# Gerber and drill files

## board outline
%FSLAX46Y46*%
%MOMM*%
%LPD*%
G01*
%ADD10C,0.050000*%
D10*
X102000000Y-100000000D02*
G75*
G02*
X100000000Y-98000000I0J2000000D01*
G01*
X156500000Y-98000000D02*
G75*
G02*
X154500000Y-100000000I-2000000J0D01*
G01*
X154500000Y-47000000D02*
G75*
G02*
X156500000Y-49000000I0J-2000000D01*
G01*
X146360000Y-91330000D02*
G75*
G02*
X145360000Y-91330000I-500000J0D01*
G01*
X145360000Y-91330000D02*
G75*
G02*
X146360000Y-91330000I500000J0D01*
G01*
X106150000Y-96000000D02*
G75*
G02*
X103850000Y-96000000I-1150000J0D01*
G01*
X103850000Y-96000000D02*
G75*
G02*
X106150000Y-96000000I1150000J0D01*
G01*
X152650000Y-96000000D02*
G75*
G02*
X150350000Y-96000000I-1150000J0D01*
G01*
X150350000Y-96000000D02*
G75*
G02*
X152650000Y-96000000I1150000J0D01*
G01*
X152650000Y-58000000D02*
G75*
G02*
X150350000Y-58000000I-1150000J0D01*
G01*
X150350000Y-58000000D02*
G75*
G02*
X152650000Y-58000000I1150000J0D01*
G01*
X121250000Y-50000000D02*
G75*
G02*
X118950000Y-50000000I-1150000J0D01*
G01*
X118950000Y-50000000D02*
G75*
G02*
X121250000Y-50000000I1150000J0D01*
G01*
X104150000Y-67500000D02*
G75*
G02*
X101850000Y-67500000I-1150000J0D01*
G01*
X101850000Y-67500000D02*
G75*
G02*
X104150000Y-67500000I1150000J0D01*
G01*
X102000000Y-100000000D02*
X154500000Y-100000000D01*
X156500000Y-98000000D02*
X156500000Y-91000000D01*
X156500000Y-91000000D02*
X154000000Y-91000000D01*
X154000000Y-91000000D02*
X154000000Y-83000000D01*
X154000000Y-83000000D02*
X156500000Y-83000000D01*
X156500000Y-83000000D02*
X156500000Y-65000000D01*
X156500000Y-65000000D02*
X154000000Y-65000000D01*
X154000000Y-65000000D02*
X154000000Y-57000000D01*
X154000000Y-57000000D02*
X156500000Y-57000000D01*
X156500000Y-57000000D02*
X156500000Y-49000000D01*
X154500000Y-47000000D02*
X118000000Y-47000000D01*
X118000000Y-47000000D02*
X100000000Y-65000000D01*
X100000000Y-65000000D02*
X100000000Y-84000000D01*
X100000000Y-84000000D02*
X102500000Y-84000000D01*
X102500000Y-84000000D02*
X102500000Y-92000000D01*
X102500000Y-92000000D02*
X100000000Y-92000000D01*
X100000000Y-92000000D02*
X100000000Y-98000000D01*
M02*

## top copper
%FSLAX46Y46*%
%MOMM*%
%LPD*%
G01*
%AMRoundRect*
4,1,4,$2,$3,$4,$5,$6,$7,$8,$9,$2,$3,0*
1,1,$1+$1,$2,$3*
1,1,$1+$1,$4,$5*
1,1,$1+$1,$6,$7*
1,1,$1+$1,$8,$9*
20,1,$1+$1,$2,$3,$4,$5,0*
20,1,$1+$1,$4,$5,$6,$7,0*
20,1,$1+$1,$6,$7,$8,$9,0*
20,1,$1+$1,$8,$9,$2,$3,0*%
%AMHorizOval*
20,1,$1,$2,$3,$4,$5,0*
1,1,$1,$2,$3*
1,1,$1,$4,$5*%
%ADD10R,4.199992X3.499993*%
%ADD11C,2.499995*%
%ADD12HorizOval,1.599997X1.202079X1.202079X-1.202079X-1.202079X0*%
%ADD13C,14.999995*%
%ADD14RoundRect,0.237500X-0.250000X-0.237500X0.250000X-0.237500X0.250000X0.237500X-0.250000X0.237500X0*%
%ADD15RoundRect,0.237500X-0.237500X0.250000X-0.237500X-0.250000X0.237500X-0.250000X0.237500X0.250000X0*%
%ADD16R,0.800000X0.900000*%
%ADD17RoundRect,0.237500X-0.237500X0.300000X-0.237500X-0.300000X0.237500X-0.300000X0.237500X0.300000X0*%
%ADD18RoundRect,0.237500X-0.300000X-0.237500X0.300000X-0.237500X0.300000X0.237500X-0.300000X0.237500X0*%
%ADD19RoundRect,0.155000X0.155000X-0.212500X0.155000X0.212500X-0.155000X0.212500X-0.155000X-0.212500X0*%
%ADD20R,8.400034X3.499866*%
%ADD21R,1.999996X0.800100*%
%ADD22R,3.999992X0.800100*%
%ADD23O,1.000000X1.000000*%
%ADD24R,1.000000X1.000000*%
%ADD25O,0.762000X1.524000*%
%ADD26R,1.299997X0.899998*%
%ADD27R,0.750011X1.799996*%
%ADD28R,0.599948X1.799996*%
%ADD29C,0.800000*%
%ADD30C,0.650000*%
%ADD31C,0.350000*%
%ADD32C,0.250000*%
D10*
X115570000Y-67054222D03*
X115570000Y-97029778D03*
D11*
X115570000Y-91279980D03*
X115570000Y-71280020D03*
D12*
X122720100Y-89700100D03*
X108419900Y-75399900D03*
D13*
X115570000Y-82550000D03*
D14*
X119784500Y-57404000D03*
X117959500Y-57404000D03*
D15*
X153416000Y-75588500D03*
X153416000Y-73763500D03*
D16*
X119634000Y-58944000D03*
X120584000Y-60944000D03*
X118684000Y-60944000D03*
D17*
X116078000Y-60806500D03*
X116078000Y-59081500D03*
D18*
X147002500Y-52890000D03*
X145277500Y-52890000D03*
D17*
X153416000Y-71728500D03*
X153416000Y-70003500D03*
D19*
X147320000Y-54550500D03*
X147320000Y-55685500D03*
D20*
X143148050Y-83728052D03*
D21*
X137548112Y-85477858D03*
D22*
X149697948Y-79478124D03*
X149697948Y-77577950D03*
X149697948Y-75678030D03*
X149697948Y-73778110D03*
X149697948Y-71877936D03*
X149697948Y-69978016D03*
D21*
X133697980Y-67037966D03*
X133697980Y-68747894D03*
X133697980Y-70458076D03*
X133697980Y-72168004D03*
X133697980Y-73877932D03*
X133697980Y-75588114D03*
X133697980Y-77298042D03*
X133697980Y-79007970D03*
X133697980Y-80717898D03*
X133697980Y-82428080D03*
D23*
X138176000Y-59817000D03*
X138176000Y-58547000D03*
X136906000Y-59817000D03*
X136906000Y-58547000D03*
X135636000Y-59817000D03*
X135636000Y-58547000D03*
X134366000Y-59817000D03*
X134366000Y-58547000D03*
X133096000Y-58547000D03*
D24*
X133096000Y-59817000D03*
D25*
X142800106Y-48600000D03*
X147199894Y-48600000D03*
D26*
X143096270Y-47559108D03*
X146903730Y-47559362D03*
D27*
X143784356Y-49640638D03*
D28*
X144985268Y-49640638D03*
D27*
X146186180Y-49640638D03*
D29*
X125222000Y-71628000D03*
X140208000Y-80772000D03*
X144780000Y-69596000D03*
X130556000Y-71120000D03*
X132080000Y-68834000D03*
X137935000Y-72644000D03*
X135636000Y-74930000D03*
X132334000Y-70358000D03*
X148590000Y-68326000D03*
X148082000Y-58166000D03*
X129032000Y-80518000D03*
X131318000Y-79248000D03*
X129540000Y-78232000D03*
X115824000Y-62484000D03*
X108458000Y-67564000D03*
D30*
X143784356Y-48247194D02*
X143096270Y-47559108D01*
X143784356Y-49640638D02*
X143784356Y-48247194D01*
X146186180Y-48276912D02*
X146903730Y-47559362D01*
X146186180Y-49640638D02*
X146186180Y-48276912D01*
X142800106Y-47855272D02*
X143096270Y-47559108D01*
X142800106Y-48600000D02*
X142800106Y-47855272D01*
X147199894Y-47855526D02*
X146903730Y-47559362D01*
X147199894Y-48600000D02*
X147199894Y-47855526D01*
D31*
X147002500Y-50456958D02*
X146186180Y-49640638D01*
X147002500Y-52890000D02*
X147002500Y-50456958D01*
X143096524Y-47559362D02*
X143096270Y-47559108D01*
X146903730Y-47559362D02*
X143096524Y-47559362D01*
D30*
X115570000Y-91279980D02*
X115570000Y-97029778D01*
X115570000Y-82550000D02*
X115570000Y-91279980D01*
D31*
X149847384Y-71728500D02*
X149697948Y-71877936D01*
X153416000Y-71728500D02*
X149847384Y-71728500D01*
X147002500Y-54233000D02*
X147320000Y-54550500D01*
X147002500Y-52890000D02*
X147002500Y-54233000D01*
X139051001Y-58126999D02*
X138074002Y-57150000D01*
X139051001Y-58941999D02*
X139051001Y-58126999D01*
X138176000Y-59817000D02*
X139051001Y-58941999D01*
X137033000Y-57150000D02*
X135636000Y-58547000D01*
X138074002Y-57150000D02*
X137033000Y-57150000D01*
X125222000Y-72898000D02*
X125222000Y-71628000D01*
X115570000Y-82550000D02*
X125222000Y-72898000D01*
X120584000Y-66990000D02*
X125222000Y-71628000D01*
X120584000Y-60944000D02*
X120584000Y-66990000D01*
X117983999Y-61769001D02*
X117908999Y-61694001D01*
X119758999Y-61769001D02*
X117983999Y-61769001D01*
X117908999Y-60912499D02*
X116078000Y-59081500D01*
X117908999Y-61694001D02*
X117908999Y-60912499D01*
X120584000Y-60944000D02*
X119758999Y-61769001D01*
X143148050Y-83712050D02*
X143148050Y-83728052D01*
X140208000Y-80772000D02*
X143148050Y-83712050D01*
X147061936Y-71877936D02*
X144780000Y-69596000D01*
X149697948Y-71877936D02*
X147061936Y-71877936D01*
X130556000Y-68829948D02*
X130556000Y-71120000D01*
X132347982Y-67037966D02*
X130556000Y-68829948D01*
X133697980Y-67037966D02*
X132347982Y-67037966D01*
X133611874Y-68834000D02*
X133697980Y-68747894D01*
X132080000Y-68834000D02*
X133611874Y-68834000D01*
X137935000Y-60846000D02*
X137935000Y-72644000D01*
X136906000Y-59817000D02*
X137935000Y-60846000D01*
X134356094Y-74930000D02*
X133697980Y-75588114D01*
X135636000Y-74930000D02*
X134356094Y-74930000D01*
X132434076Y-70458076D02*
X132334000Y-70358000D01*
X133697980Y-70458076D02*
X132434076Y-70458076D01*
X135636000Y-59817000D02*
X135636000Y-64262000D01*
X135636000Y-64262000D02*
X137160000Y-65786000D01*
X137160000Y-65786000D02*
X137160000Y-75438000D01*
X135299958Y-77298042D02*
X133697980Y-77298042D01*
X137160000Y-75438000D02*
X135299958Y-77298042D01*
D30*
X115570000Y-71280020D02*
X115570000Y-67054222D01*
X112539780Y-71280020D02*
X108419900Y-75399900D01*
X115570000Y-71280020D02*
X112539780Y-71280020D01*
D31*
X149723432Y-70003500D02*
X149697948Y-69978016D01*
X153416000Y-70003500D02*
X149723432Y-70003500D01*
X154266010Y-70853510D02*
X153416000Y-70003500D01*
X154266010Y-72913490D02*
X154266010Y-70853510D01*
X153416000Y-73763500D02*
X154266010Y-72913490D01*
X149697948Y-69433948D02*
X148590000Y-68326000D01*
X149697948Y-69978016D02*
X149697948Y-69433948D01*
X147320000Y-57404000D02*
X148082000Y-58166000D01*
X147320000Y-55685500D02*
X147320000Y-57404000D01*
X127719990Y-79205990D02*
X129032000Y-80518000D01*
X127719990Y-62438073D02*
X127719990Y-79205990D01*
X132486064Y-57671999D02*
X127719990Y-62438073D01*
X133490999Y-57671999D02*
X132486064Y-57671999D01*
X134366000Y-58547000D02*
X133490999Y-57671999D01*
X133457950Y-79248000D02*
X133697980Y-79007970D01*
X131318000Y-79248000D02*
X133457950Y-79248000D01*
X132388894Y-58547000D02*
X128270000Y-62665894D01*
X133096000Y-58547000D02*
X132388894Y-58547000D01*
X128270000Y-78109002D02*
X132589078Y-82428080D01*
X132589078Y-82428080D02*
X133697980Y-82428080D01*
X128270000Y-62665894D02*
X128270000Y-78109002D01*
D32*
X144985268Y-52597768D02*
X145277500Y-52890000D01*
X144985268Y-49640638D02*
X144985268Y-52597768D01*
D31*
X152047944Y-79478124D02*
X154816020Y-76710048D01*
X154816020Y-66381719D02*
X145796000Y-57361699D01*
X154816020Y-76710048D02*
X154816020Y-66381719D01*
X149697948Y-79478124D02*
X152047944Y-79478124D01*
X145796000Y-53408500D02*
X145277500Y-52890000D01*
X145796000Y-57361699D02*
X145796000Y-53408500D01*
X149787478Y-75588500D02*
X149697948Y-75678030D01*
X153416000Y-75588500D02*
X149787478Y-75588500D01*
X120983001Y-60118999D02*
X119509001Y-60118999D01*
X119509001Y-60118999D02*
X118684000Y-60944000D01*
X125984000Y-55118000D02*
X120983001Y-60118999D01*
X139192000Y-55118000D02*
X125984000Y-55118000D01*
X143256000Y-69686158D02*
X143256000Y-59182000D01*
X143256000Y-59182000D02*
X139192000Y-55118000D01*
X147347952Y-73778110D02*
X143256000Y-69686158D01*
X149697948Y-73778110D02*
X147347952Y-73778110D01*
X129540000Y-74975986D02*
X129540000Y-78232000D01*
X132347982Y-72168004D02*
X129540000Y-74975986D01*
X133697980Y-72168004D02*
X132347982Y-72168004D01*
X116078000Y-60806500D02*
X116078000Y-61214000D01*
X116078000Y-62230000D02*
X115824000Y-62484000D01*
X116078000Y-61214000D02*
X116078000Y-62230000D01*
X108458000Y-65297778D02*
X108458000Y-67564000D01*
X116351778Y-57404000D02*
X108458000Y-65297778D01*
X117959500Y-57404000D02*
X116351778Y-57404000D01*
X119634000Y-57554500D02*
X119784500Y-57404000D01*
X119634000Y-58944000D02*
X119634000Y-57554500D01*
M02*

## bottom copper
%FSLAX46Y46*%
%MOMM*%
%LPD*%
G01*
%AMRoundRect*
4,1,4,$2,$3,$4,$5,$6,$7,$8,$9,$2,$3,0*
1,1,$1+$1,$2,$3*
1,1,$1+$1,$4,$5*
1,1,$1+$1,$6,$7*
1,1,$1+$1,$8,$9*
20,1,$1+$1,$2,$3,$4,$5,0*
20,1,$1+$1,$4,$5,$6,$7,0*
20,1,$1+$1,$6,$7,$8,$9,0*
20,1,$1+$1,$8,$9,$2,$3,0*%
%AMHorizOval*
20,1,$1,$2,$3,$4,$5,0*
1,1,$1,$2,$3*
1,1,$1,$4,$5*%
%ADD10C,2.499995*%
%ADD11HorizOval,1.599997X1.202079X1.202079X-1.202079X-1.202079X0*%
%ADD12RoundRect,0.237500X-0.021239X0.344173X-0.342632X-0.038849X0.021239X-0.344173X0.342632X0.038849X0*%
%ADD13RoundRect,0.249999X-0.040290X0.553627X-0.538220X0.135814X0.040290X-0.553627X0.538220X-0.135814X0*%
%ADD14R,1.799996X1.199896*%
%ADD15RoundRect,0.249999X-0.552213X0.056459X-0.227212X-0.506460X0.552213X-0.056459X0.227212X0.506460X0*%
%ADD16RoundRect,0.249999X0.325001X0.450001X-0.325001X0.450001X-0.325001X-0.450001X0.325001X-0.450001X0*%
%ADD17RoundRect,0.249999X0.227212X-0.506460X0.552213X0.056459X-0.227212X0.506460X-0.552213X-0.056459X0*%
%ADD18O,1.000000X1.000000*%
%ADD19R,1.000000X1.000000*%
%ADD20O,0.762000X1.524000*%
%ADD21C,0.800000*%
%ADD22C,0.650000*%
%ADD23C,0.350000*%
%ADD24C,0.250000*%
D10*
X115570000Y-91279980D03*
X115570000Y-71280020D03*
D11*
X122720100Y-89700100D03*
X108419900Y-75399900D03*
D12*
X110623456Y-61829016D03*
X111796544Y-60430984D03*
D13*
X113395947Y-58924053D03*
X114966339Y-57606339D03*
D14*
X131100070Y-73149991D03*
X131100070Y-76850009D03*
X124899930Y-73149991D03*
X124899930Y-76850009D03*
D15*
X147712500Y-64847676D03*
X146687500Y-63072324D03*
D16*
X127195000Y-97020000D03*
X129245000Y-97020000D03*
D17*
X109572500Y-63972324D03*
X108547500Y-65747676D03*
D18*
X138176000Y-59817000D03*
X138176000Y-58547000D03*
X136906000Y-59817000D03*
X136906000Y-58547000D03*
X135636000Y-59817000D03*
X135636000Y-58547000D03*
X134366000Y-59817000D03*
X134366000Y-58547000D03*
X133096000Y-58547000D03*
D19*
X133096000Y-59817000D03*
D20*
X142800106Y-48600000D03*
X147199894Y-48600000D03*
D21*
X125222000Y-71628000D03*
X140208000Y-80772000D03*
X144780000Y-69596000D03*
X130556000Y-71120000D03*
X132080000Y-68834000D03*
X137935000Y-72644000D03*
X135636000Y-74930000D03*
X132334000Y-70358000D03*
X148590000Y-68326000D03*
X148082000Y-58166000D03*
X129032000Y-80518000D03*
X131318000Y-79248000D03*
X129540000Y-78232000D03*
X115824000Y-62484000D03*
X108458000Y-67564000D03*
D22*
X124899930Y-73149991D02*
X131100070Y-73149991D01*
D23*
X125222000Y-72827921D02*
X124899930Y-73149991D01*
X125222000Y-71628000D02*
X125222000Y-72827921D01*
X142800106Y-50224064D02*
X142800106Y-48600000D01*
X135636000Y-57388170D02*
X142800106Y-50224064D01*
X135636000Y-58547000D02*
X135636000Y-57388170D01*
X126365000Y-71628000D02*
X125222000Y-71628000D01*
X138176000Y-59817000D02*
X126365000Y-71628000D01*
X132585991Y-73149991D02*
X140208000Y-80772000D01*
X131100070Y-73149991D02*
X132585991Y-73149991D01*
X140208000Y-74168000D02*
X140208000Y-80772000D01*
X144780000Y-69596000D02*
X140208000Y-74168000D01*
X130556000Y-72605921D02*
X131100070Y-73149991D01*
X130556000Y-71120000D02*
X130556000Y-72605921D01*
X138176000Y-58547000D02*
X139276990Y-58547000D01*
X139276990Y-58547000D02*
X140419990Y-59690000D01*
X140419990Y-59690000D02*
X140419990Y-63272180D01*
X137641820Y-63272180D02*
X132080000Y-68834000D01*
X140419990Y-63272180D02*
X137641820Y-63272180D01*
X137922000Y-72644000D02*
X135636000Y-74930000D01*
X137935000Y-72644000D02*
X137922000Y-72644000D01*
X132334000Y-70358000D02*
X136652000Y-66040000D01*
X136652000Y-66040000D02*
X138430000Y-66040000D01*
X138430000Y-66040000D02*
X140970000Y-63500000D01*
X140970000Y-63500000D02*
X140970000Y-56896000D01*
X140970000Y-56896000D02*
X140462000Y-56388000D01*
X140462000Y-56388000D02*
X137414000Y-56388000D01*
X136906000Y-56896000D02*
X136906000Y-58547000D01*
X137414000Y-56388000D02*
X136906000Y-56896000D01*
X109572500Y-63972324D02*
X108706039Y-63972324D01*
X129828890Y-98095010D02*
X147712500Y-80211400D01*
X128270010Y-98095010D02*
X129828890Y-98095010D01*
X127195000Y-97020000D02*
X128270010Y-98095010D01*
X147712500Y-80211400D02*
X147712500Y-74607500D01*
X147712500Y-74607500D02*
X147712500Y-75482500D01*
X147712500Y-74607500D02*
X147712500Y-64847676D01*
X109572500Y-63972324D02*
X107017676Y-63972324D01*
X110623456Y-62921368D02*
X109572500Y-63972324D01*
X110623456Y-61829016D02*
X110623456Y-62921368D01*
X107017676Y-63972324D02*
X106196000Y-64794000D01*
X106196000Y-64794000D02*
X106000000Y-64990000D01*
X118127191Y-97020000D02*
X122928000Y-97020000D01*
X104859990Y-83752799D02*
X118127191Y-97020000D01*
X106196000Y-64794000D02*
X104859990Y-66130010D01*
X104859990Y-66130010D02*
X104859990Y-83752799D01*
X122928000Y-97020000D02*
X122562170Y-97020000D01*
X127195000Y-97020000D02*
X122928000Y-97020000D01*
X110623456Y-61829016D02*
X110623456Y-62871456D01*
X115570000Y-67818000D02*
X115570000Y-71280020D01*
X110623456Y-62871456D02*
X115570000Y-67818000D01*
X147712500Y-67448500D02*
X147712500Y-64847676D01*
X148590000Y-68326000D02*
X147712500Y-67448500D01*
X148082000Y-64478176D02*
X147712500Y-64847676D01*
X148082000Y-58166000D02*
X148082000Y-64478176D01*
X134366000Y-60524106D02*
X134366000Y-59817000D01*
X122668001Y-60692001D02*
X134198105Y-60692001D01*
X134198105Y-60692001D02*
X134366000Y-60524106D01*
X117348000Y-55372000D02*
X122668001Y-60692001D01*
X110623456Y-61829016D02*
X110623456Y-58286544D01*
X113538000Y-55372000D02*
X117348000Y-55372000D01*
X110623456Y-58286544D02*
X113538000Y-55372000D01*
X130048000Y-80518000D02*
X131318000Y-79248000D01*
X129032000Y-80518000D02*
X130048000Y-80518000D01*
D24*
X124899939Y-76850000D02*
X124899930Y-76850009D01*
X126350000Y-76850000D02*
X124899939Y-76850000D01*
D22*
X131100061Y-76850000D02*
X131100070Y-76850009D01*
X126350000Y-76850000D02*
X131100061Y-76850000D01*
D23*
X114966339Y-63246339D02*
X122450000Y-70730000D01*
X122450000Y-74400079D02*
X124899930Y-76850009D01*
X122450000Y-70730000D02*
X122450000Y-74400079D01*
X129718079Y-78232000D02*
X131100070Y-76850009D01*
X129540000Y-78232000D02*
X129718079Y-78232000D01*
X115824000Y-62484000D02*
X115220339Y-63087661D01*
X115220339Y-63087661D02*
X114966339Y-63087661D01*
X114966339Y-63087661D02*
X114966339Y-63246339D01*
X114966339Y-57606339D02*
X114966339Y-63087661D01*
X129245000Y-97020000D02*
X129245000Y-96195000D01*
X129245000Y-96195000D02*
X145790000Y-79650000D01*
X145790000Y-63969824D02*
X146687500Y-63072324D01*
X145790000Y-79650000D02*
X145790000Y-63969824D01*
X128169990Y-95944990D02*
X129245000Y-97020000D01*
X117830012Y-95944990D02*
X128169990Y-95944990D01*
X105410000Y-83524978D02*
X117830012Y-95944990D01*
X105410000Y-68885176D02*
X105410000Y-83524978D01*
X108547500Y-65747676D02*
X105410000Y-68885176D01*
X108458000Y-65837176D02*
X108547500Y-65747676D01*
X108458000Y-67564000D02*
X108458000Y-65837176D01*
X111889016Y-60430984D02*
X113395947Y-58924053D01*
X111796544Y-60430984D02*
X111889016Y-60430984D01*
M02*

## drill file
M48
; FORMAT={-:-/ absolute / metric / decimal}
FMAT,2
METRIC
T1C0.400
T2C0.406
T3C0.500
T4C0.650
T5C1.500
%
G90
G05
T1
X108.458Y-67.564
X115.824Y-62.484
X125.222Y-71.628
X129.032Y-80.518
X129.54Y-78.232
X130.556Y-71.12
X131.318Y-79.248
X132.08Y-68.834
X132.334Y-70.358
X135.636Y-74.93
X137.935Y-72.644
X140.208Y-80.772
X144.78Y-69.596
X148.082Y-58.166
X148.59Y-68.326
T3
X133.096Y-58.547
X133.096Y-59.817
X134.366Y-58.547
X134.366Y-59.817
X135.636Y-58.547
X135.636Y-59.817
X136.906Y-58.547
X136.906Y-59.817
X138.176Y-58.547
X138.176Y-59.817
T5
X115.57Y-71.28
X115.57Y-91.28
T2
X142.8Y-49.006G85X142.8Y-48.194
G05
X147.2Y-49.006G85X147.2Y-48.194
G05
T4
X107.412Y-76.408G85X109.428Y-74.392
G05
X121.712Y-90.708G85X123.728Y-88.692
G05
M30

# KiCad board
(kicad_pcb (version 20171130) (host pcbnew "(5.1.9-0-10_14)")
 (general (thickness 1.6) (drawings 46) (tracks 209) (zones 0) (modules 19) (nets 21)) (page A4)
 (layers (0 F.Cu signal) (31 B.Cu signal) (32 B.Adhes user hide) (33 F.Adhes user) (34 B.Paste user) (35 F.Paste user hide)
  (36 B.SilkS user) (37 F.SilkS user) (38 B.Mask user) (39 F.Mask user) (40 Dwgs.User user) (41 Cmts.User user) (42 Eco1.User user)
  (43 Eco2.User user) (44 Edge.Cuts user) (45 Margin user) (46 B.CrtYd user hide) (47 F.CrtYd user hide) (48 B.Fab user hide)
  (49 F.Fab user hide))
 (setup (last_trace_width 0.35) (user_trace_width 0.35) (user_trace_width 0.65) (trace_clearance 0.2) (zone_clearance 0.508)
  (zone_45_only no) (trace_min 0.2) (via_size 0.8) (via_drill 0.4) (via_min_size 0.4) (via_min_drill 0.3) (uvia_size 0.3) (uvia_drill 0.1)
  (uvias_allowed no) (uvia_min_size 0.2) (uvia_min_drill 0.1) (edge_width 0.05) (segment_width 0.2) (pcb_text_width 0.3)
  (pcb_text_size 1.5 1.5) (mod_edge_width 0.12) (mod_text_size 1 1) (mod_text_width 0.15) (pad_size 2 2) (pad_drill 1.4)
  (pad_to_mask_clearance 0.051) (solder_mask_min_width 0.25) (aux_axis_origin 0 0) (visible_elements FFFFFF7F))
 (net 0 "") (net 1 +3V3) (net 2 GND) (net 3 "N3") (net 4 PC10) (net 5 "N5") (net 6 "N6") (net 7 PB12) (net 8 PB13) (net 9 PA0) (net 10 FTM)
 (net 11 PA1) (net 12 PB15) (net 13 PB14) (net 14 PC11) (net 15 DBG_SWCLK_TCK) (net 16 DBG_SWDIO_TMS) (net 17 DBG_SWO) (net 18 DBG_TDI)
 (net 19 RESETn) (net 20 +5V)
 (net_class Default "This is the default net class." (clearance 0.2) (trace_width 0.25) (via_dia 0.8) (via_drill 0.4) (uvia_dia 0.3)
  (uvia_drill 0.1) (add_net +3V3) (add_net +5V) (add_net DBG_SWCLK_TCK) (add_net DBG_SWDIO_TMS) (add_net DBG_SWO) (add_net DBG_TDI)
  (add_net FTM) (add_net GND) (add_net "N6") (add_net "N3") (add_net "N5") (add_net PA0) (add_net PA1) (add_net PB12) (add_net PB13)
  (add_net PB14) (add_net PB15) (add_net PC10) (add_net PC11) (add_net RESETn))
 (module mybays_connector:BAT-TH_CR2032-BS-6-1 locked (layer F.Cu) (at 115.57 82.042 90)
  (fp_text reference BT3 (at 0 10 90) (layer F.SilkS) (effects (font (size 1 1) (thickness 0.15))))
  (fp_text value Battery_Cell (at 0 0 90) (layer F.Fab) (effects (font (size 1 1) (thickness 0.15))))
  (pad 1 smd rect (at 14.987778 0 90) (size 3.499993 4.199992) (layers F.Cu F.Paste F.Mask) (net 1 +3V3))
  (pad 2 smd rect (at -14.987778 0 90) (size 3.499993 4.199992) (layers F.Cu F.Paste F.Mask) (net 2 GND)))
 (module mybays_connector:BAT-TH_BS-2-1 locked (layer F.Cu) (at 115.57 81.28 180)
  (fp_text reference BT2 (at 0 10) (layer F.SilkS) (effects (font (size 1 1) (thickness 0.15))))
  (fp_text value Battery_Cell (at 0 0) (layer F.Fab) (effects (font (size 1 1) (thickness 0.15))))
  (pad 2 thru_hole circle (at 0 -9.99998 270) (size 2.499995 2.499995) (drill 1.500022) (layers *.Cu *.Mask) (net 2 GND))
  (pad 1 thru_hole circle (at 0 9.99998 270) (size 2.499995 2.499995) (drill 1.500022) (layers *.Cu *.Mask) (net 1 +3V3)))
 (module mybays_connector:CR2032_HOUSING (layer F.Cu) (at 115.57 82.55 90)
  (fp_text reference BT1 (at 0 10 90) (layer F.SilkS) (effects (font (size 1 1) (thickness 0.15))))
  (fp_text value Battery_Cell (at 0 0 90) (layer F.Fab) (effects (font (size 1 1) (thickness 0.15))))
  (pad 3 thru_hole oval (at -7.1501 7.1501 135) (size 1.599997 4.99999) (drill oval 0.649986 3.499968) (layers *.Cu *.Mask))
  (pad 1 thru_hole oval (at 7.1501 -7.1501 135) (size 1.599997 4.99999) (drill oval 0.649986 3.500044) (layers *.Cu *.Mask) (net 1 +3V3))
  (pad 2 smd circle (at 0 0 90) (size 14.999995 14.999995) (layers F.Cu F.Paste F.Mask) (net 2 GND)))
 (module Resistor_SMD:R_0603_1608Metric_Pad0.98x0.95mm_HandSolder (layer B.Cu) (at 111.21 61.13 230)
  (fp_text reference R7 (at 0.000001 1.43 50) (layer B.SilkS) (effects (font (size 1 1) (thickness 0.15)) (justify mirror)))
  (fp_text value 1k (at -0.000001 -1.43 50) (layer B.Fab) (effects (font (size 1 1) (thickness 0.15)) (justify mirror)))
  (pad 2 smd roundrect (at 0.9125 0 230) (size 0.975 0.95) (layers B.Cu B.Paste B.Mask) (roundrect_rratio 0.25) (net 1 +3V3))
  (pad 1 smd roundrect (at -0.9125 0 230) (size 0.975 0.95) (layers B.Cu B.Paste B.Mask) (roundrect_rratio 0.25) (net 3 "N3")))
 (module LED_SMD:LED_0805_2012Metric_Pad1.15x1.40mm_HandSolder (layer B.Cu) (at 114.181143 58.265196 220)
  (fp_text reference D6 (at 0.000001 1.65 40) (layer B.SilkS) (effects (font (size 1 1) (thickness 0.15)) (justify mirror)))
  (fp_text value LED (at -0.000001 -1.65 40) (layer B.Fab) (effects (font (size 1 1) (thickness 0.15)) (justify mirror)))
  (pad 2 smd roundrect (at 1.025 0 220) (size 1.15 1.4) (layers B.Cu B.Paste B.Mask) (roundrect_rratio 0.2173904347826087) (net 3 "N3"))
  (pad 1 smd roundrect (at -1.025 0 220) (size 1.15 1.4) (layers B.Cu B.Paste B.Mask) (roundrect_rratio 0.2173904347826087) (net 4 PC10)))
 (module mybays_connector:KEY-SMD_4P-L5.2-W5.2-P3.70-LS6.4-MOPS (layer B.Cu) (at 128 75)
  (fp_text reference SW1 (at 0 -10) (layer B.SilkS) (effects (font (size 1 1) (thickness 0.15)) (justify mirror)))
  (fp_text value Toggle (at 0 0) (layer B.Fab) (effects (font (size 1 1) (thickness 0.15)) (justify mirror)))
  (pad 4 smd rect (at 3.10007 -1.850009) (size 1.799996 1.199896) (layers B.Cu B.Paste B.Mask) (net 2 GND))
  (pad 3 smd rect (at 3.10007 1.850009) (size 1.799996 1.199896) (layers B.Cu B.Paste B.Mask) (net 4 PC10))
  (pad 2 smd rect (at -3.10007 -1.850009) (size 1.799996 1.199896) (layers B.Cu B.Paste B.Mask) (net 2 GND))
  (pad 1 smd rect (at -3.10007 1.850009) (size 1.799996 1.199896) (layers B.Cu B.Paste B.Mask) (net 4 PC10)))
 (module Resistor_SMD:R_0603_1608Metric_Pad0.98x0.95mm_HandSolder (layer F.Cu) (at 118.872 57.404)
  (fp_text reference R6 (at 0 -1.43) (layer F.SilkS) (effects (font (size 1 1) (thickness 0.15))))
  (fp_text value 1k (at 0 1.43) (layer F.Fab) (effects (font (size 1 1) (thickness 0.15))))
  (pad 2 smd roundrect (at 0.9125 0) (size 0.975 0.95) (layers F.Cu F.Paste F.Mask) (roundrect_rratio 0.25) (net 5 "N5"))
  (pad 1 smd roundrect (at -0.9125 0) (size 0.975 0.95) (layers F.Cu F.Paste F.Mask) (roundrect_rratio 0.25) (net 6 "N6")))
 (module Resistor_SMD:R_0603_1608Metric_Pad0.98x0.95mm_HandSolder (layer F.Cu) (at 153.416 74.676 270)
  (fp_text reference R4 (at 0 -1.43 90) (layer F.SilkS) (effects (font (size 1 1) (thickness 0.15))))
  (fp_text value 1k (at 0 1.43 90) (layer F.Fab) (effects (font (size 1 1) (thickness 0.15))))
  (pad 2 smd roundrect (at 0.9125 0 270) (size 0.975 0.95) (layers F.Cu F.Paste F.Mask) (roundrect_rratio 0.25) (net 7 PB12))
  (pad 1 smd roundrect (at -0.9125 0 270) (size 0.975 0.95) (layers F.Cu F.Paste F.Mask) (roundrect_rratio 0.25) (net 1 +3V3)))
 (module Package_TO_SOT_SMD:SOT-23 (layer F.Cu) (at 119.634 59.944 90)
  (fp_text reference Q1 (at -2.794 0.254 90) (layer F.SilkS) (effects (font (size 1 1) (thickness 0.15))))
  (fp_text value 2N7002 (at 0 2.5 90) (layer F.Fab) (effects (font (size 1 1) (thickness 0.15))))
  (pad 3 smd rect (at 1 0 90) (size 0.9 0.8) (layers F.Cu F.Paste F.Mask) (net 5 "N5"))
  (pad 2 smd rect (at -1 0.95 90) (size 0.9 0.8) (layers F.Cu F.Paste F.Mask) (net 2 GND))
  (pad 1 smd rect (at -1 -0.95 90) (size 0.9 0.8) (layers F.Cu F.Paste F.Mask) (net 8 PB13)))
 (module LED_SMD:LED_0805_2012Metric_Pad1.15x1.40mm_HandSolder (layer B.Cu) (at 147.2 63.96 300)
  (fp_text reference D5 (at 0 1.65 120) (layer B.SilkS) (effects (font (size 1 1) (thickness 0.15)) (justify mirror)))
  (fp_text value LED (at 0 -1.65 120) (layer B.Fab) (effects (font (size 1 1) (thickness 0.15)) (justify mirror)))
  (pad 2 smd roundrect (at 1.025 0 300) (size 1.15 1.4) (layers B.Cu B.Paste B.Mask) (roundrect_rratio 0.2173904347826087) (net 1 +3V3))
  (pad 1 smd roundrect (at -1.025 0 300) (size 1.15 1.4) (layers B.Cu B.Paste B.Mask) (roundrect_rratio 0.2173904347826087) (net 6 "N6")))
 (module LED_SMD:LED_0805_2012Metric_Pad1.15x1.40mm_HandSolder (layer B.Cu) (at 128.22 97.02 180)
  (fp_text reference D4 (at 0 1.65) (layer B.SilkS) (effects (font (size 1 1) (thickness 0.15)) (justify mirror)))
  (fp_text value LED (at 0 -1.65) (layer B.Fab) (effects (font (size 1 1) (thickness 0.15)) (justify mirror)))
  (pad 2 smd roundrect (at 1.025 0 180) (size 1.15 1.4) (layers B.Cu B.Paste B.Mask) (roundrect_rratio 0.2173904347826087) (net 1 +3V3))
  (pad 1 smd roundrect (at -1.025 0 180) (size 1.15 1.4) (layers B.Cu B.Paste B.Mask) (roundrect_rratio 0.2173904347826087) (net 6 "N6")))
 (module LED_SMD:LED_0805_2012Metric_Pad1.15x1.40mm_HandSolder (layer B.Cu) (at 109.06 64.86 60)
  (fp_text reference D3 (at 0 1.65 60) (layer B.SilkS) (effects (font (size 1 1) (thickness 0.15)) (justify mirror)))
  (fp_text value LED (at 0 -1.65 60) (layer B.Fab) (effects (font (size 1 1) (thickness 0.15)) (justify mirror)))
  (pad 2 smd roundrect (at 1.025 0 60) (size 1.15 1.4) (layers B.Cu B.Paste B.Mask) (roundrect_rratio 0.2173904347826087) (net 1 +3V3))
  (pad 1 smd roundrect (at -1.025 0 60) (size 1.15 1.4) (layers B.Cu B.Paste B.Mask) (roundrect_rratio 0.2173904347826087) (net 6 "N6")))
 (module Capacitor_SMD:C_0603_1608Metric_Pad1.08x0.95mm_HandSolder (layer F.Cu) (at 116.078 59.944 270)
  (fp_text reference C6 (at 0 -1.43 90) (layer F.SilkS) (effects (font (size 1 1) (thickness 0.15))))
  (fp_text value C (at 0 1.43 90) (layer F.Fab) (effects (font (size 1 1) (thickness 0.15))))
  (pad 2 smd roundrect (at 0.8625 0 270) (size 1.075 0.95) (layers F.Cu F.Paste F.Mask) (roundrect_rratio 0.25) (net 4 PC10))
  (pad 1 smd roundrect (at -0.8625 0 270) (size 1.075 0.95) (layers F.Cu F.Paste F.Mask) (roundrect_rratio 0.25) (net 2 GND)))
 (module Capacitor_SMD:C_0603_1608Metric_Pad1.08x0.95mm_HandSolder (layer F.Cu) (at 146.14 52.89)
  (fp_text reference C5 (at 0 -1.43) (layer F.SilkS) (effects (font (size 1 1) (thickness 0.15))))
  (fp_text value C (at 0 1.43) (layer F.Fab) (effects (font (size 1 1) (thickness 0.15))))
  (pad 2 smd roundrect (at 0.8625 0) (size 1.075 0.95) (layers F.Cu F.Paste F.Mask) (roundrect_rratio 0.25) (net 2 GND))
  (pad 1 smd roundrect (at -0.8625 0) (size 1.075 0.95) (layers F.Cu F.Paste F.Mask) (roundrect_rratio 0.25) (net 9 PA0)))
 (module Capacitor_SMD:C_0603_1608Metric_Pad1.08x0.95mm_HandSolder (layer F.Cu) (at 153.416 70.866 270)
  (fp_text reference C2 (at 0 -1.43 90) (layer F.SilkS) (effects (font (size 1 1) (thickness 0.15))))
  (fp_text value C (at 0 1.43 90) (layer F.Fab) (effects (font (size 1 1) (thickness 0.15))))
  (pad 2 smd roundrect (at 0.8625 0 270) (size 1.075 0.95) (layers F.Cu F.Paste F.Mask) (roundrect_rratio 0.25) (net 2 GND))
  (pad 1 smd roundrect (at -0.8625 0 270) (size 1.075 0.95) (layers F.Cu F.Paste F.Mask) (roundrect_rratio 0.25) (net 1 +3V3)))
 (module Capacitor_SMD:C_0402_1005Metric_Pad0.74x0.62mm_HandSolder (layer F.Cu) (at 147.32 55.118 90)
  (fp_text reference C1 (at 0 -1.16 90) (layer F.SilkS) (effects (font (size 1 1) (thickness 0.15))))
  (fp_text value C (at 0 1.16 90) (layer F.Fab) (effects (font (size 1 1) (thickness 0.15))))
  (pad 2 smd roundrect (at 0.5675 0 90) (size 0.735 0.62) (layers F.Cu F.Paste F.Mask) (roundrect_rratio 0.25) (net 2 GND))
  (pad 1 smd roundrect (at -0.5675 0 90) (size 0.735 0.62) (layers F.Cu F.Paste F.Mask) (roundrect_rratio 0.25) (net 1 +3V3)))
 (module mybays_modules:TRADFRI (layer F.Cu) (at 142.748 77.978 270)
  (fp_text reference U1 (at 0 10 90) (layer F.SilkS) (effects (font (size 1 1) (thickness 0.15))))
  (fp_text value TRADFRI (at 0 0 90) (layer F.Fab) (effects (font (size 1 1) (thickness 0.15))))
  (pad 18 smd rect (at 5.750052 -0.40005 180) (size 8.400034 3.499866) (layers F.Cu F.Paste F.Mask) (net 2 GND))
  (pad 17 smd rect (at 7.499858 5.199888 180) (size 1.999996 0.8001) (layers F.Cu F.Paste F.Mask) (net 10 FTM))
  (pad 16 smd rect (at 1.500124 -6.949948 180) (size 3.999992 0.8001) (layers F.Cu F.Paste F.Mask) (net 9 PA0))
  (pad 15 smd rect (at -0.40005 -6.949948 180) (size 3.999992 0.8001) (layers F.Cu F.Paste F.Mask) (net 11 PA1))
  (pad 14 smd rect (at -2.29997 -6.949948 180) (size 3.999992 0.8001) (layers F.Cu F.Paste F.Mask) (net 7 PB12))
  (pad 13 smd rect (at -4.19989 -6.949948 180) (size 3.999992 0.8001) (layers F.Cu F.Paste F.Mask) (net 8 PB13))
  (pad 12 smd rect (at -6.100064 -6.949948 180) (size 3.999992 0.8001) (layers F.Cu F.Paste F.Mask) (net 2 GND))
  (pad 11 smd rect (at -7.999984 -6.949948 180) (size 3.999992 0.8001) (layers F.Cu F.Paste F.Mask) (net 1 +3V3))
  (pad 1 smd rect (at -10.940034 9.05002 180) (size 1.999996 0.8001) (layers F.Cu F.Paste F.Mask) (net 2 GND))
  (pad 2 smd rect (at -9.230106 9.05002 180) (size 1.999996 0.8001) (layers F.Cu F.Paste F.Mask) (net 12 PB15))
  (pad 3 smd rect (at -7.519924 9.05002 180) (size 1.999996 0.8001) (layers F.Cu F.Paste F.Mask) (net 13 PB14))
  (pad 4 smd rect (at -5.809996 9.05002 180) (size 1.999996 0.8001) (layers F.Cu F.Paste F.Mask) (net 4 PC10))
  (pad 5 smd rect (at -4.100068 9.05002 180) (size 1.999996 0.8001) (layers F.Cu F.Paste F.Mask) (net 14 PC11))
  (pad 6 smd rect (at -2.389886 9.05002 180) (size 1.999996 0.8001) (layers F.Cu F.Paste F.Mask) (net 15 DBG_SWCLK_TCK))
  (pad 7 smd rect (at -0.679958 9.05002 180) (size 1.999996 0.8001) (layers F.Cu F.Paste F.Mask) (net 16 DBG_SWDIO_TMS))
  (pad 8 smd rect (at 1.02997 9.05002 180) (size 1.999996 0.8001) (layers F.Cu F.Paste F.Mask) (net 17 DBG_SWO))
  (pad 9 smd rect (at 2.739898 9.05002 180) (size 1.999996 0.8001) (layers F.Cu F.Paste F.Mask) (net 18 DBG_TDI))
  (pad 10 smd rect (at 4.45008 9.05002 180) (size 1.999996 0.8001) (layers F.Cu F.Paste F.Mask) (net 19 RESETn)))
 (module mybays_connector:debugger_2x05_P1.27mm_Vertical (layer F.Cu) (at 135.636 59.182 90)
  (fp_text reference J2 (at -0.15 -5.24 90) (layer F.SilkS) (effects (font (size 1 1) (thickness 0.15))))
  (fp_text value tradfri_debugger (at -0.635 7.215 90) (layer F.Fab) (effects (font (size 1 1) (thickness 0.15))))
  (pad 9 thru_hole oval (at -0.635 2.54 90) (size 1 1) (drill 0.5) (layers *.Cu *.Mask) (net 2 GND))
  (pad 10 thru_hole oval (at 0.635 2.54 90) (size 1 1) (drill 0.5) (layers *.Cu *.Mask) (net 12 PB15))
  (pad 7 thru_hole oval (at -0.635 1.27 90) (size 1 1) (drill 0.5) (layers *.Cu *.Mask) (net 15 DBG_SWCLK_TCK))
  (pad 8 thru_hole oval (at 0.635 1.27 90) (size 1 1) (drill 0.5) (layers *.Cu *.Mask) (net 13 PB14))
  (pad 5 thru_hole oval (at -0.635 0 90) (size 1 1) (drill 0.5) (layers *.Cu *.Mask) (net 16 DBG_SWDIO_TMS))
  (pad 6 thru_hole oval (at 0.635 0 90) (size 1 1) (drill 0.5) (layers *.Cu *.Mask) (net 2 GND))
  (pad 3 thru_hole oval (at -0.635 -1.27 90) (size 1 1) (drill 0.5) (layers *.Cu *.Mask) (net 1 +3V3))
  (pad 4 thru_hole oval (at 0.635 -1.27 90) (size 1 1) (drill 0.5) (layers *.Cu *.Mask) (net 17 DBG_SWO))
  (pad 2 thru_hole oval (at 0.635 -2.54 90) (size 1 1) (drill 0.5) (layers *.Cu *.Mask) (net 19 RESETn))
  (pad 1 thru_hole rect (at -0.635 -2.54 90) (size 1 1) (drill 0.5) (layers *.Cu *.Mask) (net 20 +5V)))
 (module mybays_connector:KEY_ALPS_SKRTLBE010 (layer F.Cu) (at 145 48.6 180)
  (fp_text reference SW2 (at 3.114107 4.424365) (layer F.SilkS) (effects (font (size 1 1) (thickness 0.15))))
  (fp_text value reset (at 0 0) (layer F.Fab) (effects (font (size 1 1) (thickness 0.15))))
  (pad 4 thru_hole oval (at 2.199894 0 180) (size 0.762 1.524) (drill oval 0.4064 1.2192) (layers *.Cu *.Mask) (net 2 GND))
  (pad 4 thru_hole oval (at -2.199894 0 180) (size 0.762 1.524) (drill oval 0.4064 1.2192) (layers *.Cu *.Mask) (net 2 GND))
  (pad 4 smd rect (at 1.90373 1.040892 270) (size 0.899998 1.299997) (layers F.Cu F.Paste F.Mask) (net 2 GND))
  (pad 4 smd rect (at -1.90373 1.040638 270) (size 0.899998 1.299997) (layers F.Cu F.Paste F.Mask) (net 2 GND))
  (pad 3 smd rect (at 1.215644 -1.040638 180) (size 0.750011 1.799996) (layers F.Cu F.Paste F.Mask) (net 2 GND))
  (pad 2 smd rect (at 0.014732 -1.040638 180) (size 0.599948 1.799996) (layers F.Cu F.Paste F.Mask) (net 9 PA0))
  (pad 1 smd rect (at -1.18618 -1.040638 180) (size 0.750011 1.799996) (layers F.Cu F.Paste F.Mask) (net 2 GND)))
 (gr_arc (start 102 98) (end 100 98) (angle -90) (layer Edge.Cuts) (width 0.05))
 (gr_arc (start 154.5 98) (end 154.5 100) (angle -90) (layer Edge.Cuts) (width 0.05))
 (gr_arc (start 154.5 49) (end 156.5 49) (angle -90) (layer Edge.Cuts) (width 0.05))
 (gr_circle (center 145.86 91.33) (end 146.36 91.33) (layer Edge.Cuts) (width 0.05))
 (gr_circle (center 105 96) (end 105 97.15) (layer Edge.Cuts) (width 0.05))
 (gr_circle (center 151.5 96) (end 151.5 97.15) (layer Edge.Cuts) (width 0.05))
 (gr_circle (center 151.5 58) (end 151.5 59.15) (layer Edge.Cuts) (width 0.05))
 (gr_circle (center 120.1 50) (end 120.1 51.15) (layer Edge.Cuts) (width 0.05))
 (gr_circle (center 103 67.5) (end 103 68.65) (layer Edge.Cuts) (width 0.05))
 (gr_line (start 102 100) (end 154.5 100) (layer Edge.Cuts) (width 0.05))
 (gr_line (start 156.5 98) (end 156.5 91) (layer Edge.Cuts) (width 0.05))
 (gr_line (start 156.5 91) (end 154 91) (layer Edge.Cuts) (width 0.05))
 (gr_line (start 154 91) (end 154 83) (layer Edge.Cuts) (width 0.05))
 (gr_line (start 154 83) (end 156.5 83) (layer Edge.Cuts) (width 0.05))
 (gr_line (start 156.5 83) (end 156.5 65) (layer Edge.Cuts) (width 0.05))
 (gr_line (start 156.5 65) (end 154 65) (layer Edge.Cuts) (width 0.05))
 (gr_line (start 154 65) (end 154 57) (layer Edge.Cuts) (width 0.05))
 (gr_line (start 154 57) (end 156.5 57) (layer Edge.Cuts) (width 0.05))
 (gr_line (start 156.5 57) (end 156.5 49) (layer Edge.Cuts) (width 0.05))
 (gr_line (start 154.5 47) (end 118 47) (layer Edge.Cuts) (width 0.05))
 (gr_line (start 118 47) (end 100 65) (layer Edge.Cuts) (width 0.05))
 (gr_line (start 100 65) (end 100 84) (layer Edge.Cuts) (width 0.05))
 (gr_line (start 100 84) (end 102.5 84) (layer Edge.Cuts) (width 0.05))
 (gr_line (start 102.5 84) (end 102.5 92) (layer Edge.Cuts) (width 0.05))
 (gr_line (start 102.5 92) (end 100 92) (layer Edge.Cuts) (width 0.05))
 (gr_line (start 100 92) (end 100 98) (layer Edge.Cuts) (width 0.05))
 (segment (start 143.784356 48.247194) (end 143.09627 47.559108) (width 0.65) (layer F.Cu) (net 2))
 (segment (start 143.784356 49.640638) (end 143.784356 48.247194) (width 0.65) (layer F.Cu) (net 2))
 (segment (start 146.18618 48.276912) (end 146.90373 47.559362) (width 0.65) (layer F.Cu) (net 2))
 (segment (start 146.18618 49.640638) (end 146.18618 48.276912) (width 0.65) (layer F.Cu) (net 2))
 (segment (start 142.800106 47.855272) (end 143.09627 47.559108) (width 0.65) (layer F.Cu) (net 2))
 (segment (start 142.800106 48.6) (end 142.800106 47.855272) (width 0.65) (layer F.Cu) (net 2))
 (segment (start 147.199894 47.855526) (end 146.90373 47.559362) (width 0.65) (layer F.Cu) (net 2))
 (segment (start 147.199894 48.6) (end 147.199894 47.855526) (width 0.65) (layer F.Cu) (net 2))
 (segment (start 147.0025 50.456958) (end 146.18618 49.640638) (width 0.35) (layer F.Cu) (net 2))
 (segment (start 147.0025 52.89) (end 147.0025 50.456958) (width 0.35) (layer F.Cu) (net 2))
 (segment (start 143.096524 47.559362) (end 143.09627 47.559108) (width 0.35) (layer F.Cu) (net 2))
 (segment (start 146.90373 47.559362) (end 143.096524 47.559362) (width 0.35) (layer F.Cu) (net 2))
 (segment (start 124.89993 73.149991) (end 131.10007 73.149991) (width 0.65) (layer B.Cu) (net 2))
 (segment (start 115.57 91.27998) (end 115.57 97.029778) (width 0.65) (layer F.Cu) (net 2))
 (segment (start 115.57 82.55) (end 115.57 91.27998) (width 0.65) (layer F.Cu) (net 2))
 (segment (start 149.847384 71.7285) (end 149.697948 71.877936) (width 0.35) (layer F.Cu) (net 2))
 (segment (start 153.416 71.7285) (end 149.847384 71.7285) (width 0.35) (layer F.Cu) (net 2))
 (segment (start 147.0025 54.233) (end 147.32 54.5505) (width 0.35) (layer F.Cu) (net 2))
 (segment (start 147.0025 52.89) (end 147.0025 54.233) (width 0.35) (layer F.Cu) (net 2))
 (segment (start 139.051001 58.126999) (end 138.074002 57.15) (width 0.35) (layer F.Cu) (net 2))
 (segment (start 139.051001 58.941999) (end 139.051001 58.126999) (width 0.35) (layer F.Cu) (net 2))
 (segment (start 138.176 59.817) (end 139.051001 58.941999) (width 0.35) (layer F.Cu) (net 2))
 (segment (start 137.033 57.15) (end 135.636 58.547) (width 0.35) (layer F.Cu) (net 2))
 (segment (start 138.074002 57.15) (end 137.033 57.15) (width 0.35) (layer F.Cu) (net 2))
 (via (at 125.222 71.628) (size 0.8) (drill 0.4) (layers F.Cu B.Cu) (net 2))
 (segment (start 125.222 72.898) (end 125.222 71.628) (width 0.35) (layer F.Cu) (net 2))
 (segment (start 115.57 82.55) (end 125.222 72.898) (width 0.35) (layer F.Cu) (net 2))
 (segment (start 125.222 72.827921) (end 124.89993 73.149991) (width 0.35) (layer B.Cu) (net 2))
 (segment (start 125.222 71.628) (end 125.222 72.827921) (width 0.35) (layer B.Cu) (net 2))
 (segment (start 120.584 66.99) (end 125.222 71.628) (width 0.35) (layer F.Cu) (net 2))
 (segment (start 120.584 60.944) (end 120.584 66.99) (width 0.35) (layer F.Cu) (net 2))
 (segment (start 117.983999 61.769001) (end 117.908999 61.694001) (width 0.35) (layer F.Cu) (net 2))
 (segment (start 119.758999 61.769001) (end 117.983999 61.769001) (width 0.35) (layer F.Cu) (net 2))
 (segment (start 117.908999 60.912499) (end 116.078 59.0815) (width 0.35) (layer F.Cu) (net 2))
 (segment (start 117.908999 61.694001) (end 117.908999 60.912499) (width 0.35) (layer F.Cu) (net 2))
 (segment (start 120.584 60.944) (end 119.758999 61.769001) (width 0.35) (layer F.Cu) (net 2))
 (segment (start 142.800106 50.224064) (end 142.800106 48.6) (width 0.35) (layer B.Cu) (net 2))
 (segment (start 135.636 57.38817) (end 142.800106 50.224064) (width 0.35) (layer B.Cu) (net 2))
 (segment (start 135.636 58.547) (end 135.636 57.38817) (width 0.35) (layer B.Cu) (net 2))
 (segment (start 126.365 71.628) (end 125.222 71.628) (width 0.35) (layer B.Cu) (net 2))
 (segment (start 138.176 59.817) (end 126.365 71.628) (width 0.35) (layer B.Cu) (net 2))
 (via (at 140.208 80.772) (size 0.8) (drill 0.4) (layers F.Cu B.Cu) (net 2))
 (segment (start 132.585991 73.149991) (end 140.208 80.772) (width 0.35) (layer B.Cu) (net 2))
 (segment (start 131.10007 73.149991) (end 132.585991 73.149991) (width 0.35) (layer B.Cu) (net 2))
 (segment (start 143.14805 83.71205) (end 143.14805 83.728052) (width 0.35) (layer F.Cu) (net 2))
 (segment (start 140.208 80.772) (end 143.14805 83.71205) (width 0.35) (layer F.Cu) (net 2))
 (via (at 144.78 69.596) (size 0.8) (drill 0.4) (layers F.Cu B.Cu) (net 2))
 (segment (start 147.061936 71.877936) (end 144.78 69.596) (width 0.35) (layer F.Cu) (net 2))
 (segment (start 149.697948 71.877936) (end 147.061936 71.877936) (width 0.35) (layer F.Cu) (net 2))
 (segment (start 140.208 74.168) (end 140.208 80.772) (width 0.35) (layer B.Cu) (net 2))
 (segment (start 144.78 69.596) (end 140.208 74.168) (width 0.35) (layer B.Cu) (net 2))
 (via (at 130.556 71.12) (size 0.8) (drill 0.4) (layers F.Cu B.Cu) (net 2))
 (segment (start 130.556 68.829948) (end 130.556 71.12) (width 0.35) (layer F.Cu) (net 2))
 (segment (start 132.347982 67.037966) (end 130.556 68.829948) (width 0.35) (layer F.Cu) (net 2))
 (segment (start 133.69798 67.037966) (end 132.347982 67.037966) (width 0.35) (layer F.Cu) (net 2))
 (segment (start 130.556 72.605921) (end 131.10007 73.149991) (width 0.35) (layer B.Cu) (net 2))
 (segment (start 130.556 71.12) (end 130.556 72.605921) (width 0.35) (layer B.Cu) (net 2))
 (segment (start 138.176 58.547) (end 139.27699 58.547) (width 0.35) (layer B.Cu) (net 12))
 (segment (start 139.27699 58.547) (end 140.41999 59.69) (width 0.35) (layer B.Cu) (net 12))
 (segment (start 140.41999 59.69) (end 140.41999 63.27218) (width 0.35) (layer B.Cu) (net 12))
 (via (at 132.08 68.834) (size 0.8) (drill 0.4) (layers F.Cu B.Cu) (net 12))
 (segment (start 137.64182 63.27218) (end 132.08 68.834) (width 0.35) (layer B.Cu) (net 12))
 (segment (start 140.41999 63.27218) (end 137.64182 63.27218) (width 0.35) (layer B.Cu) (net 12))
 (segment (start 133.611874 68.834) (end 133.69798 68.747894) (width 0.35) (layer F.Cu) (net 12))
 (segment (start 132.08 68.834) (end 133.611874 68.834) (width 0.35) (layer F.Cu) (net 12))
 (via (at 137.935 72.644) (size 0.8) (drill 0.4) (layers F.Cu B.Cu) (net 15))
 (segment (start 137.935 60.846) (end 137.935 72.644) (width 0.35) (layer F.Cu) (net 15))
 (segment (start 136.906 59.817) (end 137.935 60.846) (width 0.35) (layer F.Cu) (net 15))
 (via (at 135.636 74.93) (size 0.8) (drill 0.4) (layers F.Cu B.Cu) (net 15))
 (segment (start 137.922 72.644) (end 135.636 74.93) (width 0.35) (layer B.Cu) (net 15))
 (segment (start 137.935 72.644) (end 137.922 72.644) (width 0.35) (layer B.Cu) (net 15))
 (segment (start 134.356094 74.93) (end 133.69798 75.588114) (width 0.35) (layer F.Cu) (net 15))
 (segment (start 135.636 74.93) (end 134.356094 74.93) (width 0.35) (layer F.Cu) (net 15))
 (via (at 132.334 70.358) (size 0.8) (drill 0.4) (layers F.Cu B.Cu) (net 13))
 (segment (start 132.434076 70.458076) (end 132.334 70.358) (width 0.35) (layer F.Cu) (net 13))
 (segment (start 133.69798 70.458076) (end 132.434076 70.458076) (width 0.35) (layer F.Cu) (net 13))
 (segment (start 132.334 70.358) (end 136.652 66.04) (width 0.35) (layer B.Cu) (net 13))
 (segment (start 136.652 66.04) (end 138.43 66.04) (width 0.35) (layer B.Cu) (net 13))
 (segment (start 138.43 66.04) (end 140.97 63.5) (width 0.35) (layer B.Cu) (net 13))
 (segment (start 140.97 63.5) (end 140.97 56.896) (width 0.35) (layer B.Cu) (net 13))
 (segment (start 140.97 56.896) (end 140.462 56.388) (width 0.35) (layer B.Cu) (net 13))
 (segment (start 140.462 56.388) (end 137.414 56.388) (width 0.35) (layer B.Cu) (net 13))
 (segment (start 136.906 56.896) (end 136.906 58.547) (width 0.35) (layer B.Cu) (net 13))
 (segment (start 137.414 56.388) (end 136.906 56.896) (width 0.35) (layer B.Cu) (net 13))
 (segment (start 135.636 59.817) (end 135.636 64.262) (width 0.35) (layer F.Cu) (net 16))
 (segment (start 135.636 64.262) (end 137.16 65.786) (width 0.35) (layer F.Cu) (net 16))
 (segment (start 137.16 65.786) (end 137.16 75.438) (width 0.35) (layer F.Cu) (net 16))
 (segment (start 135.299958 77.298042) (end 133.69798 77.298042) (width 0.35) (layer F.Cu) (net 16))
 (segment (start 137.16 75.438) (end 135.299958 77.298042) (width 0.35) (layer F.Cu) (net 16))
 (segment (start 109.5725 63.972324) (end 108.706039 63.972324) (width 0.35) (layer B.Cu) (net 1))
 (segment (start 129.82889 98.09501) (end 147.7125 80.2114) (width 0.35) (layer B.Cu) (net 1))
 (segment (start 128.27001 98.09501) (end 129.82889 98.09501) (width 0.35) (layer B.Cu) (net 1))
 (segment (start 127.195 97.02) (end 128.27001 98.09501) (width 0.35) (layer B.Cu) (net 1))
 (segment (start 147.7125 80.2114) (end 147.7125 74.6075) (width 0.35) (layer B.Cu) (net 1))
 (segment (start 147.7125 74.6075) (end 147.7125 75.4825) (width 0.35) (layer B.Cu) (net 1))
 (segment (start 147.7125 74.6075) (end 147.7125 64.847676) (width 0.35) (layer B.Cu) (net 1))
 (segment (start 109.5725 63.972324) (end 107.017676 63.972324) (width 0.35) (layer B.Cu) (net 1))
 (segment (start 110.623456 62.921368) (end 109.5725 63.972324) (width 0.35) (layer B.Cu) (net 1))
 (segment (start 110.623456 61.829016) (end 110.623456 62.921368) (width 0.35) (layer B.Cu) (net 1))
 (segment (start 107.017676 63.972324) (end 106.196 64.794) (width 0.35) (layer B.Cu) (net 1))
 (segment (start 106.196 64.794) (end 106 64.99) (width 0.35) (layer B.Cu) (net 1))
 (segment (start 118.127191 97.02) (end 122.928 97.02) (width 0.35) (layer B.Cu) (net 1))
 (segment (start 104.85999 83.752799) (end 118.127191 97.02) (width 0.35) (layer B.Cu) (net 1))
 (segment (start 106.196 64.794) (end 104.85999 66.13001) (width 0.35) (layer B.Cu) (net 1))
 (segment (start 104.85999 66.13001) (end 104.85999 83.752799) (width 0.35) (layer B.Cu) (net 1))
 (segment (start 122.928 97.02) (end 122.56217 97.02) (width 0.35) (layer B.Cu) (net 1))
 (segment (start 127.195 97.02) (end 122.928 97.02) (width 0.35) (layer B.Cu) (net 1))
 (segment (start 115.57 71.28002) (end 115.57 67.054222) (width 0.65) (layer F.Cu) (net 1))
 (segment (start 112.53978 71.28002) (end 108.4199 75.3999) (width 0.65) (layer F.Cu) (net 1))
 (segment (start 115.57 71.28002) (end 112.53978 71.28002) (width 0.65) (layer F.Cu) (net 1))
 (segment (start 149.723432 70.0035) (end 149.697948 69.978016) (width 0.35) (layer F.Cu) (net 1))
 (segment (start 153.416 70.0035) (end 149.723432 70.0035) (width 0.35) (layer F.Cu) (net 1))
 (segment (start 154.26601 70.85351) (end 153.416 70.0035) (width 0.35) (layer F.Cu) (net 1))
 (segment (start 154.26601 72.91349) (end 154.26601 70.85351) (width 0.35) (layer F.Cu) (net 1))
 (segment (start 153.416 73.7635) (end 154.26601 72.91349) (width 0.35) (layer F.Cu) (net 1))
 (segment (start 110.623456 61.829016) (end 110.623456 62.871456) (width 0.35) (layer B.Cu) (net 1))
 (segment (start 115.57 67.818) (end 115.57 71.28002) (width 0.35) (layer B.Cu) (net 1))
 (segment (start 110.623456 62.871456) (end 115.57 67.818) (width 0.35) (layer B.Cu) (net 1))
 (via (at 148.59 68.326) (size 0.8) (drill 0.4) (layers F.Cu B.Cu) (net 1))
 (segment (start 149.697948 69.433948) (end 148.59 68.326) (width 0.35) (layer F.Cu) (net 1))
 (segment (start 149.697948 69.978016) (end 149.697948 69.433948) (width 0.35) (layer F.Cu) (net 1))
 (segment (start 147.7125 67.4485) (end 147.7125 64.847676) (width 0.35) (layer B.Cu) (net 1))
 (segment (start 148.59 68.326) (end 147.7125 67.4485) (width 0.35) (layer B.Cu) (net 1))
 (via (at 148.082 58.166) (size 0.8) (drill 0.4) (layers F.Cu B.Cu) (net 1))
 (segment (start 147.32 57.404) (end 148.082 58.166) (width 0.35) (layer F.Cu) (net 1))
 (segment (start 147.32 55.6855) (end 147.32 57.404) (width 0.35) (layer F.Cu) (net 1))
 (segment (start 148.082 64.478176) (end 147.7125 64.847676) (width 0.35) (layer B.Cu) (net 1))
 (segment (start 148.082 58.166) (end 148.082 64.478176) (width 0.35) (layer B.Cu) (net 1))
 (segment (start 134.366 60.524106) (end 134.366 59.817) (width 0.35) (layer B.Cu) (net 1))
 (segment (start 122.668001 60.692001) (end 134.198105 60.692001) (width 0.35) (layer B.Cu) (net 1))
 (segment (start 134.198105 60.692001) (end 134.366 60.524106) (width 0.35) (layer B.Cu) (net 1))
 (segment (start 117.348 55.372) (end 122.668001 60.692001) (width 0.35) (layer B.Cu) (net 1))
 (segment (start 110.623456 61.829016) (end 110.623456 58.286544) (width 0.35) (layer B.Cu) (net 1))
 (segment (start 113.538 55.372) (end 117.348 55.372) (width 0.35) (layer B.Cu) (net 1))
 (segment (start 110.623456 58.286544) (end 113.538 55.372) (width 0.35) (layer B.Cu) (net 1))
 (via (at 129.032 80.518) (size 0.8) (drill 0.4) (layers F.Cu B.Cu) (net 17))
 (segment (start 127.71999 79.20599) (end 129.032 80.518) (width 0.35) (layer F.Cu) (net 17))
 (segment (start 127.71999 62.438073) (end 127.71999 79.20599) (width 0.35) (layer F.Cu) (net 17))
 (segment (start 132.486064 57.671999) (end 127.71999 62.438073) (width 0.35) (layer F.Cu) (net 17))
 (segment (start 133.490999 57.671999) (end 132.486064 57.671999) (width 0.35) (layer F.Cu) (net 17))
 (segment (start 134.366 58.547) (end 133.490999 57.671999) (width 0.35) (layer F.Cu) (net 17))
 (via (at 131.318 79.248) (size 0.8) (drill 0.4) (layers F.Cu B.Cu) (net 17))
 (segment (start 130.048 80.518) (end 131.318 79.248) (width 0.35) (layer B.Cu) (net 17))
 (segment (start 129.032 80.518) (end 130.048 80.518) (width 0.35) (layer B.Cu) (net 17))
 (segment (start 133.45795 79.248) (end 133.69798 79.00797) (width 0.35) (layer F.Cu) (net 17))
 (segment (start 131.318 79.248) (end 133.45795 79.248) (width 0.35) (layer F.Cu) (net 17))
 (segment (start 132.388894 58.547) (end 128.27 62.665894) (width 0.35) (layer F.Cu) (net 19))
 (segment (start 133.096 58.547) (end 132.388894 58.547) (width 0.35) (layer F.Cu) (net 19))
 (segment (start 128.27 78.109002) (end 132.589078 82.42808) (width 0.35) (layer F.Cu) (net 19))
 (segment (start 132.589078 82.42808) (end 133.69798 82.42808) (width 0.35) (layer F.Cu) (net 19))
 (segment (start 128.27 62.665894) (end 128.27 78.109002) (width 0.35) (layer F.Cu) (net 19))
 (segment (start 144.985268 52.597768) (end 145.2775 52.89) (width 0.25) (layer F.Cu) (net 9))
 (segment (start 144.985268 49.640638) (end 144.985268 52.597768) (width 0.25) (layer F.Cu) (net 9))
 (segment (start 152.047944 79.478124) (end 154.81602 76.710048) (width 0.35) (layer F.Cu) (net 9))
 (segment (start 154.81602 66.381719) (end 145.796 57.361699) (width 0.35) (layer F.Cu) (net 9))
 (segment (start 154.81602 76.710048) (end 154.81602 66.381719) (width 0.35) (layer F.Cu) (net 9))
 (segment (start 149.697948 79.478124) (end 152.047944 79.478124) (width 0.35) (layer F.Cu) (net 9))
 (segment (start 145.796 53.4085) (end 145.2775 52.89) (width 0.35) (layer F.Cu) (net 9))
 (segment (start 145.796 57.361699) (end 145.796 53.4085) (width 0.35) (layer F.Cu) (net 9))
 (segment (start 149.787478 75.5885) (end 149.697948 75.67803) (width 0.35) (layer F.Cu) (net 7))
 (segment (start 153.416 75.5885) (end 149.787478 75.5885) (width 0.35) (layer F.Cu) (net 7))
 (segment (start 120.983001 60.118999) (end 119.509001 60.118999) (width 0.35) (layer F.Cu) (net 8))
 (segment (start 119.509001 60.118999) (end 118.684 60.944) (width 0.35) (layer F.Cu) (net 8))
 (segment (start 125.984 55.118) (end 120.983001 60.118999) (width 0.35) (layer F.Cu) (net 8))
 (segment (start 139.192 55.118) (end 125.984 55.118) (width 0.35) (layer F.Cu) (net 8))
 (segment (start 143.256 69.686158) (end 143.256 59.182) (width 0.35) (layer F.Cu) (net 8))
 (segment (start 143.256 59.182) (end 139.192 55.118) (width 0.35) (layer F.Cu) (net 8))
 (segment (start 147.347952 73.77811) (end 143.256 69.686158) (width 0.35) (layer F.Cu) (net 8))
 (segment (start 149.697948 73.77811) (end 147.347952 73.77811) (width 0.35) (layer F.Cu) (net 8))
 (segment (start 124.899939 76.85) (end 124.89993 76.850009) (width 0.25) (layer B.Cu) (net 4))
 (segment (start 126.35 76.85) (end 124.899939 76.85) (width 0.25) (layer B.Cu) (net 4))
 (segment (start 131.100061 76.85) (end 131.10007 76.850009) (width 0.65) (layer B.Cu) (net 4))
 (segment (start 126.35 76.85) (end 131.100061 76.85) (width 0.65) (layer B.Cu) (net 4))
 (segment (start 114.966339 63.246339) (end 122.45 70.73) (width 0.35) (layer B.Cu) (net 4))
 (segment (start 122.45 74.400079) (end 124.89993 76.850009) (width 0.35) (layer B.Cu) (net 4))
 (segment (start 122.45 70.73) (end 122.45 74.400079) (width 0.35) (layer B.Cu) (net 4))
 (via (at 129.54 78.232) (size 0.8) (drill 0.4) (layers F.Cu B.Cu) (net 4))
 (segment (start 129.54 74.975986) (end 129.54 78.232) (width 0.35) (layer F.Cu) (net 4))
 (segment (start 132.347982 72.168004) (end 129.54 74.975986) (width 0.35) (layer F.Cu) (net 4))
 (segment (start 133.69798 72.168004) (end 132.347982 72.168004) (width 0.35) (layer F.Cu) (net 4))
 (segment (start 129.718079 78.232) (end 131.10007 76.850009) (width 0.35) (layer B.Cu) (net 4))
 (segment (start 129.54 78.232) (end 129.718079 78.232) (width 0.35) (layer B.Cu) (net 4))
 (segment (start 116.078 60.8065) (end 116.078 61.214) (width 0.35) (layer F.Cu) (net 4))
 (via (at 115.824 62.484) (size 0.8) (drill 0.4) (layers F.Cu B.Cu) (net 4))
 (segment (start 116.078 62.23) (end 115.824 62.484) (width 0.35) (layer F.Cu) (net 4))
 (segment (start 116.078 61.214) (end 116.078 62.23) (width 0.35) (layer F.Cu) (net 4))
 (segment (start 115.824 62.484) (end 115.220339 63.087661) (width 0.35) (layer B.Cu) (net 4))
 (segment (start 115.220339 63.087661) (end 114.966339 63.087661) (width 0.35) (layer B.Cu) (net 4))
 (segment (start 114.966339 63.087661) (end 114.966339 63.246339) (width 0.35) (layer B.Cu) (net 4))
 (segment (start 114.966339 57.606339) (end 114.966339 63.087661) (width 0.35) (layer B.Cu) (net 4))
 (segment (start 129.245 97.02) (end 129.245 96.195) (width 0.35) (layer B.Cu) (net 6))
 (segment (start 129.245 96.195) (end 145.79 79.65) (width 0.35) (layer B.Cu) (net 6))
 (segment (start 145.79 63.969824) (end 146.6875 63.072324) (width 0.35) (layer B.Cu) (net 6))
 (segment (start 145.79 79.65) (end 145.79 63.969824) (width 0.35) (layer B.Cu) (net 6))
 (segment (start 128.16999 95.94499) (end 129.245 97.02) (width 0.35) (layer B.Cu) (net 6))
 (segment (start 117.830012 95.94499) (end 128.16999 95.94499) (width 0.35) (layer B.Cu) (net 6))
 (segment (start 105.41 83.524978) (end 117.830012 95.94499) (width 0.35) (layer B.Cu) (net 6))
 (segment (start 105.41 68.885176) (end 105.41 83.524978) (width 0.35) (layer B.Cu) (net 6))
 (segment (start 108.5475 65.747676) (end 105.41 68.885176) (width 0.35) (layer B.Cu) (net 6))
 (segment (start 108.458 65.297778) (end 108.458 67.564) (width 0.35) (layer F.Cu) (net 6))
 (segment (start 116.351778 57.404) (end 108.458 65.297778) (width 0.35) (layer F.Cu) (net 6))
 (via (at 108.458 67.564) (size 0.8) (drill 0.4) (layers F.Cu B.Cu) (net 6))
 (segment (start 117.9595 57.404) (end 116.351778 57.404) (width 0.35) (layer F.Cu) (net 6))
 (segment (start 108.458 65.837176) (end 108.5475 65.747676) (width 0.35) (layer B.Cu) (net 6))
 (segment (start 108.458 67.564) (end 108.458 65.837176) (width 0.35) (layer B.Cu) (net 6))
 (segment (start 119.634 57.5545) (end 119.7845 57.404) (width 0.35) (layer F.Cu) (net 5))
 (segment (start 119.634 58.944) (end 119.634 57.5545) (width 0.35) (layer F.Cu) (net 5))
 (segment (start 111.889016 60.430984) (end 113.395947 58.924053) (width 0.35) (layer B.Cu) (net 3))
 (segment (start 111.796544 60.430984) (end 111.889016 60.430984) (width 0.35) (layer B.Cu) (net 3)))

